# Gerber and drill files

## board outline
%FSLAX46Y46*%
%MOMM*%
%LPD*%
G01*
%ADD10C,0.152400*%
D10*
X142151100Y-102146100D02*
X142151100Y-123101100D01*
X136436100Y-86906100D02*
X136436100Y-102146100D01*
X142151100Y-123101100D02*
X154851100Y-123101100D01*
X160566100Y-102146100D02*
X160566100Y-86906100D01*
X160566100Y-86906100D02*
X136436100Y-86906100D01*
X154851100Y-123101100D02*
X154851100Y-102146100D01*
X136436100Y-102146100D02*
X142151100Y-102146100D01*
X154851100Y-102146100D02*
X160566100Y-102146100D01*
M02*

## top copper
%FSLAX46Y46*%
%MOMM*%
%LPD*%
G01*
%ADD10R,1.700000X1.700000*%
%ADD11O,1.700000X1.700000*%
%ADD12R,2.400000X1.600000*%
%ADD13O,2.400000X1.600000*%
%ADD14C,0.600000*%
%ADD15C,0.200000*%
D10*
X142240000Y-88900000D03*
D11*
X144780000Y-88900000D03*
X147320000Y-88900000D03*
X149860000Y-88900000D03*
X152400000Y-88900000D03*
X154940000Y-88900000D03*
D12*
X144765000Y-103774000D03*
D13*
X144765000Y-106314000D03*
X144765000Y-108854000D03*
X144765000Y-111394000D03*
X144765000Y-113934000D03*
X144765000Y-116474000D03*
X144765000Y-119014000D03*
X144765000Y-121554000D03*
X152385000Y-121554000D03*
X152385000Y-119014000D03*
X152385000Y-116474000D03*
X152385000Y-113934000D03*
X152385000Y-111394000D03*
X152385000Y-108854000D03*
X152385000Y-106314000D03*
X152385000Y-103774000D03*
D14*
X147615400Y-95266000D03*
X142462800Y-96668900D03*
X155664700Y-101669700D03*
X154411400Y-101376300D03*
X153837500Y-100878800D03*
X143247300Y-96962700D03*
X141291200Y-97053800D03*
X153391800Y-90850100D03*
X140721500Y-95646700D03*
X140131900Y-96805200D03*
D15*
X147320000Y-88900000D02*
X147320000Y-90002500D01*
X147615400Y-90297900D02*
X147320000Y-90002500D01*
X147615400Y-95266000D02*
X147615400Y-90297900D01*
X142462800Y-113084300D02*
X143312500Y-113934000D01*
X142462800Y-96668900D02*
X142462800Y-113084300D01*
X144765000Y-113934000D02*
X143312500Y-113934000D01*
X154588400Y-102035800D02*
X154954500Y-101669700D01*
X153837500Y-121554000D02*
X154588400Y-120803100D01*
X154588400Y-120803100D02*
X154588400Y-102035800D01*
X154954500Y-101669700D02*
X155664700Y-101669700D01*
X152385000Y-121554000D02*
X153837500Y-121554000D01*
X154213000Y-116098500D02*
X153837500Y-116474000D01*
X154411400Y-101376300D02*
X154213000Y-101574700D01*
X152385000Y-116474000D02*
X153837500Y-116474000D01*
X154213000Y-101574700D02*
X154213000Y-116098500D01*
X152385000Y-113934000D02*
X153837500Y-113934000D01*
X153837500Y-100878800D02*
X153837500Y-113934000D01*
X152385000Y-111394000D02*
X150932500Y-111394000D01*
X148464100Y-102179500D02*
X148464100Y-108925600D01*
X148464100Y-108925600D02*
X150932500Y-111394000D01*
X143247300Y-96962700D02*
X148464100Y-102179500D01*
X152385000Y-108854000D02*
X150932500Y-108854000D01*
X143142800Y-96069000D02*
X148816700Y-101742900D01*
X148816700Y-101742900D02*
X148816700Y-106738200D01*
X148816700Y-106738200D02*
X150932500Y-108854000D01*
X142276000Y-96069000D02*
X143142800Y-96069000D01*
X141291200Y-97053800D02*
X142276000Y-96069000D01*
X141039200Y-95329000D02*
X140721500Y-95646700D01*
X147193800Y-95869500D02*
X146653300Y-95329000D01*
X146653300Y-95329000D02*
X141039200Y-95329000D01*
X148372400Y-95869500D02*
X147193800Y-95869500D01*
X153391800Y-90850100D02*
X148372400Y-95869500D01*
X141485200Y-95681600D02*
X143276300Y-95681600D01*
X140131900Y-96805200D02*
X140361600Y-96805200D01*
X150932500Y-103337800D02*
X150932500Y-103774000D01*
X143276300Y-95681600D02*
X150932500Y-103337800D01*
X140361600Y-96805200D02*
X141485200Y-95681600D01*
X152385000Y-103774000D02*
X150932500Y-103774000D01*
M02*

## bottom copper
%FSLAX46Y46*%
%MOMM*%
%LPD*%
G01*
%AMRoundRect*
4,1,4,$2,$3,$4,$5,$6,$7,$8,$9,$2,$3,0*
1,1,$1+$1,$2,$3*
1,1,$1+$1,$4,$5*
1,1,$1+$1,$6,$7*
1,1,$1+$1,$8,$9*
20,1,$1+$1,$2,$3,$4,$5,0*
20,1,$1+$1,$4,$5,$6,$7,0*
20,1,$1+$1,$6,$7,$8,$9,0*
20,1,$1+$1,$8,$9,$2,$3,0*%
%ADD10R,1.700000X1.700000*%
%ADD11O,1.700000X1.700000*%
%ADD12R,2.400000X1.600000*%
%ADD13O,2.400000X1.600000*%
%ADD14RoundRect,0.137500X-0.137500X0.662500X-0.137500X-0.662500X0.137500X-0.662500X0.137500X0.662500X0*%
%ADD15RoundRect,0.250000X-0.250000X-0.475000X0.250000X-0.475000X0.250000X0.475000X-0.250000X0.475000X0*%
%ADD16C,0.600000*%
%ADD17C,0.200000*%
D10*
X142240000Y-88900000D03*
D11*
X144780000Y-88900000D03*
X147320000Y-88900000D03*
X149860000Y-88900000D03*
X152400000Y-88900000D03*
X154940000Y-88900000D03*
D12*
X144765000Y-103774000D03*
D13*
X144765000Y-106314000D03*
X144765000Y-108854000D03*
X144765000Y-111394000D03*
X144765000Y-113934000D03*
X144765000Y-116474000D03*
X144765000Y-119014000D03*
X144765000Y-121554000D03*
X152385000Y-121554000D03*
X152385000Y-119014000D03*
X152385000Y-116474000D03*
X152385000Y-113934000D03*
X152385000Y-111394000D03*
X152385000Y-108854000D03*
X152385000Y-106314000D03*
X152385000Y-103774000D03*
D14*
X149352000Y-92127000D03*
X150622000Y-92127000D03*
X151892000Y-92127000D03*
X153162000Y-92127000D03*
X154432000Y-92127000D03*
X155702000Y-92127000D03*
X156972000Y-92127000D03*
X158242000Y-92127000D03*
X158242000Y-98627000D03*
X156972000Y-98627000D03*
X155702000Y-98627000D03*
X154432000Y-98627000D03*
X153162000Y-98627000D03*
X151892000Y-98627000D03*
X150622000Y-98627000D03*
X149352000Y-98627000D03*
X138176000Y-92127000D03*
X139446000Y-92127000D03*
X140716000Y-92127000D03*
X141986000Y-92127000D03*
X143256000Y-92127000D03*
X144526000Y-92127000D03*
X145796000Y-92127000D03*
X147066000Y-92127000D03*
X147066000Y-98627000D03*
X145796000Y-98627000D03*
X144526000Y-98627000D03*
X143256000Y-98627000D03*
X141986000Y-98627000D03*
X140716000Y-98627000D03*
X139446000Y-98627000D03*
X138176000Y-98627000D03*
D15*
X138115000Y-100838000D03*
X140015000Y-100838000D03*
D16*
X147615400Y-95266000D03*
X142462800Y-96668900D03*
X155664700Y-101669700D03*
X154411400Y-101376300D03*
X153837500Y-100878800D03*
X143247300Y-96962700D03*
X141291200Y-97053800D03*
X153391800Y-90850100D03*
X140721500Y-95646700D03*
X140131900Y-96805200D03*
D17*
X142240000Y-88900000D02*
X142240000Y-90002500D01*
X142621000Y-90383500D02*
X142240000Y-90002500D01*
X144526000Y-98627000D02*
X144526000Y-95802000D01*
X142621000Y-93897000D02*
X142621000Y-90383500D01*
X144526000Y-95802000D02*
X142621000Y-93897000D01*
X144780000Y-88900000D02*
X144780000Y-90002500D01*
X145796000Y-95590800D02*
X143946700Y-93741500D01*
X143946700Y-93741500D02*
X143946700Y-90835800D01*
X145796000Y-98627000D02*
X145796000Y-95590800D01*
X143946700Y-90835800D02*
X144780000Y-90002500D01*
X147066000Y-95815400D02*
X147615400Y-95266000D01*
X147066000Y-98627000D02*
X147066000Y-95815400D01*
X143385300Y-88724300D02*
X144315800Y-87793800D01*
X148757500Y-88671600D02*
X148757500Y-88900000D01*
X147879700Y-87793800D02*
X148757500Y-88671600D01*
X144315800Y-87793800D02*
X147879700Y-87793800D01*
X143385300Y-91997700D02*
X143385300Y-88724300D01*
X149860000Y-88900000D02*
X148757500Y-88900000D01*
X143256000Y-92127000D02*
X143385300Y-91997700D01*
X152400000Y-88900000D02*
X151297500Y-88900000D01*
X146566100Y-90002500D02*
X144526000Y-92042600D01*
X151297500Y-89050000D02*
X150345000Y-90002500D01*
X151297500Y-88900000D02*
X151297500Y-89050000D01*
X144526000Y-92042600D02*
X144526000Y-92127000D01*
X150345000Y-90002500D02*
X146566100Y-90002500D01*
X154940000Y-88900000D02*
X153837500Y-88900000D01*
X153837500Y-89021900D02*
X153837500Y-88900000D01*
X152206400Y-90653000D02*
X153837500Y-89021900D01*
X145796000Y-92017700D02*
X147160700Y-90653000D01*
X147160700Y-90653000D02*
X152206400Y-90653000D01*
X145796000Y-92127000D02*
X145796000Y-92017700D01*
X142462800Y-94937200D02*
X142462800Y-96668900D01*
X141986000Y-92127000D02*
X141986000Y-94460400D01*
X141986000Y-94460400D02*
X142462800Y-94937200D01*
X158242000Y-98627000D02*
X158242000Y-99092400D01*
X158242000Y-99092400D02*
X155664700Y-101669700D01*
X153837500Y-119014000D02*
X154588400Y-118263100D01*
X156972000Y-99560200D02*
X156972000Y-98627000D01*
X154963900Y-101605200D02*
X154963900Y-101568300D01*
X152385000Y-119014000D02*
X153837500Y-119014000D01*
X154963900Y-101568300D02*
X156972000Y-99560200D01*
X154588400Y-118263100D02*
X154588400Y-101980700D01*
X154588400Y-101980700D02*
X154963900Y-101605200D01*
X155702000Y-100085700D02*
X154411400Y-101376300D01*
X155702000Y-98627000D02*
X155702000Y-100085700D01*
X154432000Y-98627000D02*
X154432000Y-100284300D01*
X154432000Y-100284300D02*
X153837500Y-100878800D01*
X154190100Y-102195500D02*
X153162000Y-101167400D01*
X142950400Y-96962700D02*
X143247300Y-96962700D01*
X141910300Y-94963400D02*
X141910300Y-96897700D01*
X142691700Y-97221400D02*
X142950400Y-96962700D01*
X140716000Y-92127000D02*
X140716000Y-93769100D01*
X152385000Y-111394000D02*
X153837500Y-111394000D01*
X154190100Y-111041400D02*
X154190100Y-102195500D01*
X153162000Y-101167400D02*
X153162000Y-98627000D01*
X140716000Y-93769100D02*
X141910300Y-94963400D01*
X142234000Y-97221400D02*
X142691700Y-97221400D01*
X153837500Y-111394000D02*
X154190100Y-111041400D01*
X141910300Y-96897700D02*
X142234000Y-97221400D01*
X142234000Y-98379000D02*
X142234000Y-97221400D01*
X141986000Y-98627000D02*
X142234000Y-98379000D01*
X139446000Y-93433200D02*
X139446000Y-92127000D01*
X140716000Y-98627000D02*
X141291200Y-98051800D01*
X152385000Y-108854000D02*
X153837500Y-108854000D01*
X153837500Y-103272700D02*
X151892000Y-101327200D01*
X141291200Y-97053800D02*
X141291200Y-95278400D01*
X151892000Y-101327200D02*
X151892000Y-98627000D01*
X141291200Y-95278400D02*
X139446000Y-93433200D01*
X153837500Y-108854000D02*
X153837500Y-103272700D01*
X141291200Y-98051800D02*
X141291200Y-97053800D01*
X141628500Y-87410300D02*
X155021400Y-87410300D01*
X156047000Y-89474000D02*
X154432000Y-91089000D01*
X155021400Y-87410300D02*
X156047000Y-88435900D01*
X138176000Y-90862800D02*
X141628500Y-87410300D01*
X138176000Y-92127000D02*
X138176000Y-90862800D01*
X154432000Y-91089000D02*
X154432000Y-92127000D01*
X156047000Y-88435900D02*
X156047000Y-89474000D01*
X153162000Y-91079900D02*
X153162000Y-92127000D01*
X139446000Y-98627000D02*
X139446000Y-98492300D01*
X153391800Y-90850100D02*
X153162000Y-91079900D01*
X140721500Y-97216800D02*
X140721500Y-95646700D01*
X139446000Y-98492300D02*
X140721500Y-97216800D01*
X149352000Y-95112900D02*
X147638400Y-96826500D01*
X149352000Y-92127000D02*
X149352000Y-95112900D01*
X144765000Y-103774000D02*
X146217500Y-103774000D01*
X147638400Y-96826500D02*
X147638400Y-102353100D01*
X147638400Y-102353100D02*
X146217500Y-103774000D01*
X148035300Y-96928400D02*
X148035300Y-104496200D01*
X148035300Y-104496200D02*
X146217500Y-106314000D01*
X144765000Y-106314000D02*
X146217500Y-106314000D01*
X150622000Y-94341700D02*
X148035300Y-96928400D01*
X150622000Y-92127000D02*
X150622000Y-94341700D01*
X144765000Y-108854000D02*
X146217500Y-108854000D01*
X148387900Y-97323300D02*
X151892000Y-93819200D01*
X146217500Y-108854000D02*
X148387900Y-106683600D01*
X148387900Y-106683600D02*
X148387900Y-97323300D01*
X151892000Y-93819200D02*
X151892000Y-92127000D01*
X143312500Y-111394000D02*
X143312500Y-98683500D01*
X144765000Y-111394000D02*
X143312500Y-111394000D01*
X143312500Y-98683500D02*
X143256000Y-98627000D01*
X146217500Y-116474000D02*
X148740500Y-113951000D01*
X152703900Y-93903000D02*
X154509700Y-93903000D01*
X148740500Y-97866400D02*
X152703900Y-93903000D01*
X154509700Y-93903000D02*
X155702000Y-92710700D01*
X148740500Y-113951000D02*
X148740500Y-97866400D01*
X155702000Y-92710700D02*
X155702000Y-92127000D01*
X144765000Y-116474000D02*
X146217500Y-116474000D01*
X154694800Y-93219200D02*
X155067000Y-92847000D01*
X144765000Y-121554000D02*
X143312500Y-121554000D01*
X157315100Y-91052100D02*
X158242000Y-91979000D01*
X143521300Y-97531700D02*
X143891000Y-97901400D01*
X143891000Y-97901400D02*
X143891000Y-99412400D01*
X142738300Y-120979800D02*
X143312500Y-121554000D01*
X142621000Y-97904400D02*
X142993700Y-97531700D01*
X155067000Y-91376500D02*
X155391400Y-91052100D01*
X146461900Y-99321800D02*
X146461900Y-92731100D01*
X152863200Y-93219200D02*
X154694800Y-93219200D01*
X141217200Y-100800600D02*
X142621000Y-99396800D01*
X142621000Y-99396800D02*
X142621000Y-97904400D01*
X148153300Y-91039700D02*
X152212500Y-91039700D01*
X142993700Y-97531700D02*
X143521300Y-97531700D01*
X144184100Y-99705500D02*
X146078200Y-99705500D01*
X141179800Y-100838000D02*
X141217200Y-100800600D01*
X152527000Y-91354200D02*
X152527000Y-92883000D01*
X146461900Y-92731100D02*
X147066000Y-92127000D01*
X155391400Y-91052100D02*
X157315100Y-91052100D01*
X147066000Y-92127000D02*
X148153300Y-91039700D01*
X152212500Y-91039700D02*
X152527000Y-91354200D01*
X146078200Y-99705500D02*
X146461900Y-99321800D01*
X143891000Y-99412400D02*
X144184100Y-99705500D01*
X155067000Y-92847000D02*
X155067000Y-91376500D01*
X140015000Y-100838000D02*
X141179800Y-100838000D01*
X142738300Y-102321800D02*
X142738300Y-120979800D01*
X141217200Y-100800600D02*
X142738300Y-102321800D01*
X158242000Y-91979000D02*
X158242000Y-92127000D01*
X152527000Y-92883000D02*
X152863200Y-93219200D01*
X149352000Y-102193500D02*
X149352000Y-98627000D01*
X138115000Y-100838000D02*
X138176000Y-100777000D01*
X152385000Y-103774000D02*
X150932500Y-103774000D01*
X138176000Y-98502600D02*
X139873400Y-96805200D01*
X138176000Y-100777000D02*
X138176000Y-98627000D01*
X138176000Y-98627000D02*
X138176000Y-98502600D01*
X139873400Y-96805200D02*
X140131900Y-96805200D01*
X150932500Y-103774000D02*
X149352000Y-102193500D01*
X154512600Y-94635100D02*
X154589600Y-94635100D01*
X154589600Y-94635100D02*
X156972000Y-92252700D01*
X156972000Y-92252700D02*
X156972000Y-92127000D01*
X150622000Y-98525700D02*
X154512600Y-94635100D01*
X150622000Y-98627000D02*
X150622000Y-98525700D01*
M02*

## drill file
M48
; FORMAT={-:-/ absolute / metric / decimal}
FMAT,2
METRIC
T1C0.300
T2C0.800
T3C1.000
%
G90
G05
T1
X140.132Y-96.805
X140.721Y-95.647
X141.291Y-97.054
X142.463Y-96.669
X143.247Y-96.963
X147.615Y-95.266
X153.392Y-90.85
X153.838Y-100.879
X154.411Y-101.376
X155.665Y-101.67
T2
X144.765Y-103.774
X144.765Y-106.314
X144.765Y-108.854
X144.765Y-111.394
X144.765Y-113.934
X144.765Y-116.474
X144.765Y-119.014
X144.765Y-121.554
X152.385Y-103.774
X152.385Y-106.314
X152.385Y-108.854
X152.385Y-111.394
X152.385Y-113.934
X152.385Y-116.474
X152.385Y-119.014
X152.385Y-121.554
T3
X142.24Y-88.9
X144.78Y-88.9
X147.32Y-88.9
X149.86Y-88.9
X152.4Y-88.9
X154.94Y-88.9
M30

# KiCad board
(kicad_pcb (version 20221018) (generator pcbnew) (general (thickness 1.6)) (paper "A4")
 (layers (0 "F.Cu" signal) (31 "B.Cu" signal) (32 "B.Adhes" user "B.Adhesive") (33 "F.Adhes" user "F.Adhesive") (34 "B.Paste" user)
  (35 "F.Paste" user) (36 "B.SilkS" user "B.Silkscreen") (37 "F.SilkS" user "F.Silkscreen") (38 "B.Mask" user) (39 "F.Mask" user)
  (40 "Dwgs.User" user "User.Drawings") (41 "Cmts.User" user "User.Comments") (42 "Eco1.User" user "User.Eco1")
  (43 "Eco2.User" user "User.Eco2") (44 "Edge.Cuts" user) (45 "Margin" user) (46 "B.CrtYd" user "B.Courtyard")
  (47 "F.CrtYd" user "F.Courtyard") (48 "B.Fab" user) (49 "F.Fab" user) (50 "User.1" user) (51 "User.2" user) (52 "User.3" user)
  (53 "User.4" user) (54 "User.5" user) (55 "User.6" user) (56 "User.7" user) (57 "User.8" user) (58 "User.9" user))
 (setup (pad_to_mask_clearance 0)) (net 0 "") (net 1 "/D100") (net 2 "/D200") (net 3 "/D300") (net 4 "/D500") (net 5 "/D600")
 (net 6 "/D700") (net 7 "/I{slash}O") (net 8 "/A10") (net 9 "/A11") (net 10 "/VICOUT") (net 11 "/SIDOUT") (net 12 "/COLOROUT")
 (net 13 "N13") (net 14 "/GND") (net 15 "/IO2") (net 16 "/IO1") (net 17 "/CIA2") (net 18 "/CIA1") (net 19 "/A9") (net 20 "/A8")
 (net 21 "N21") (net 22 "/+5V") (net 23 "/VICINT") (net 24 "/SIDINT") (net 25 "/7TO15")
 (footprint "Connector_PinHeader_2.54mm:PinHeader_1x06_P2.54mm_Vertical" (layer "F.Cu") (at 142.24 88.9 90)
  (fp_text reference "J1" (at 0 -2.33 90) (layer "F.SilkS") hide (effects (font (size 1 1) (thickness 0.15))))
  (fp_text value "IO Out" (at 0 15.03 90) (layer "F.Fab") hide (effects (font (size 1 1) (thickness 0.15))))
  (pad "1" thru_hole rect (at 0 0 90) (size 1.7 1.7) (drill 1) (layers "*.Cu" "*.Mask") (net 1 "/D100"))
  (pad "2" thru_hole oval (at 0 2.54 90) (size 1.7 1.7) (drill 1) (layers "*.Cu" "*.Mask") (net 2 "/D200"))
  (pad "3" thru_hole oval (at 0 5.08 90) (size 1.7 1.7) (drill 1) (layers "*.Cu" "*.Mask") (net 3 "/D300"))
  (pad "4" thru_hole oval (at 0 7.62 90) (size 1.7 1.7) (drill 1) (layers "*.Cu" "*.Mask") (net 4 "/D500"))
  (pad "5" thru_hole oval (at 0 10.16 90) (size 1.7 1.7) (drill 1) (layers "*.Cu" "*.Mask") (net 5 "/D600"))
  (pad "6" thru_hole oval (at 0 12.7 90) (size 1.7 1.7) (drill 1) (layers "*.Cu" "*.Mask") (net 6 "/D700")))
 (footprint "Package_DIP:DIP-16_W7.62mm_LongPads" (layer "F.Cu") (at 144.765 103.774)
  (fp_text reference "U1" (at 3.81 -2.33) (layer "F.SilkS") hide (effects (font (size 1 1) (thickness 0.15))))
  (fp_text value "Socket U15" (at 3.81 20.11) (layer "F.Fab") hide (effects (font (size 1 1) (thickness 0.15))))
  (pad "1" thru_hole rect (at 0 0) (size 2.4 1.6) (drill 0.8) (layers "*.Cu" "*.Mask") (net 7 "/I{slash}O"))
  (pad "2" thru_hole oval (at 0 2.54) (size 2.4 1.6) (drill 0.8) (layers "*.Cu" "*.Mask") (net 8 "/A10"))
  (pad "3" thru_hole oval (at 0 5.08) (size 2.4 1.6) (drill 0.8) (layers "*.Cu" "*.Mask") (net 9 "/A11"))
  (pad "4" thru_hole oval (at 0 7.62) (size 2.4 1.6) (drill 0.8) (layers "*.Cu" "*.Mask") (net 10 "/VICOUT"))
  (pad "5" thru_hole oval (at 0 10.16) (size 2.4 1.6) (drill 0.8) (layers "*.Cu" "*.Mask") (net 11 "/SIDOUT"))
  (pad "6" thru_hole oval (at 0 12.7) (size 2.4 1.6) (drill 0.8) (layers "*.Cu" "*.Mask") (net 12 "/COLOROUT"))
  (pad "7" thru_hole oval (at 0 15.24) (size 2.4 1.6) (drill 0.8) (layers "*.Cu" "*.Mask") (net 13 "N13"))
  (pad "8" thru_hole oval (at 0 17.78) (size 2.4 1.6) (drill 0.8) (layers "*.Cu" "*.Mask") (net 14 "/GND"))
  (pad "9" thru_hole oval (at 7.62 17.78) (size 2.4 1.6) (drill 0.8) (layers "*.Cu" "*.Mask") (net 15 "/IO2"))
  (pad "10" thru_hole oval (at 7.62 15.24) (size 2.4 1.6) (drill 0.8) (layers "*.Cu" "*.Mask") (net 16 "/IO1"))
  (pad "11" thru_hole oval (at 7.62 12.7) (size 2.4 1.6) (drill 0.8) (layers "*.Cu" "*.Mask") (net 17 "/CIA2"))
  (pad "12" thru_hole oval (at 7.62 10.16) (size 2.4 1.6) (drill 0.8) (layers "*.Cu" "*.Mask") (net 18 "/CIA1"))
  (pad "13" thru_hole oval (at 7.62 7.62) (size 2.4 1.6) (drill 0.8) (layers "*.Cu" "*.Mask") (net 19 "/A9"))
  (pad "14" thru_hole oval (at 7.62 5.08) (size 2.4 1.6) (drill 0.8) (layers "*.Cu" "*.Mask") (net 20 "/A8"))
  (pad "15" thru_hole oval (at 7.62 2.54) (size 2.4 1.6) (drill 0.8) (layers "*.Cu" "*.Mask") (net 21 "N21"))
  (pad "16" thru_hole oval (at 7.62 0) (size 2.4 1.6) (drill 0.8) (layers "*.Cu" "*.Mask") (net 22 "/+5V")))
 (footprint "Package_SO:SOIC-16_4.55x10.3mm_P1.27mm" (layer "B.Cu") (at 153.797 95.377 -90)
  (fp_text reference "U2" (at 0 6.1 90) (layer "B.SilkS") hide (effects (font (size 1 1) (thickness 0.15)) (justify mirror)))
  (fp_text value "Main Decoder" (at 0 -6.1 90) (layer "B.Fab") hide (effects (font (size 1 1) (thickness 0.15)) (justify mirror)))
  (pad "1" smd roundrect (at -3.25 4.445 270) (size 1.6 0.55) (layers "B.Cu" "B.Paste" "B.Mask") (roundrect_rratio 0.25)
   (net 7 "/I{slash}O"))
  (pad "2" smd roundrect (at -3.25 3.175 270) (size 1.6 0.55) (layers "B.Cu" "B.Paste" "B.Mask") (roundrect_rratio 0.25) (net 8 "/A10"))
  (pad "3" smd roundrect (at -3.25 1.905 270) (size 1.6 0.55) (layers "B.Cu" "B.Paste" "B.Mask") (roundrect_rratio 0.25) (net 9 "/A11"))
  (pad "4" smd roundrect (at -3.25 0.635 270) (size 1.6 0.55) (layers "B.Cu" "B.Paste" "B.Mask") (roundrect_rratio 0.25) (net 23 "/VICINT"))
  (pad "5" smd roundrect (at -3.25 -0.635 270) (size 1.6 0.55) (layers "B.Cu" "B.Paste" "B.Mask") (roundrect_rratio 0.25) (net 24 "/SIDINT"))
  (pad "6" smd roundrect (at -3.25 -1.905 270) (size 1.6 0.55) (layers "B.Cu" "B.Paste" "B.Mask") (roundrect_rratio 0.25)
   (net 12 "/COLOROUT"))
  (pad "7" smd roundrect (at -3.25 -3.175 270) (size 1.6 0.55) (layers "B.Cu" "B.Paste" "B.Mask") (roundrect_rratio 0.25) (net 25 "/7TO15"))
  (pad "8" smd roundrect (at -3.25 -4.445 270) (size 1.6 0.55) (layers "B.Cu" "B.Paste" "B.Mask") (roundrect_rratio 0.25) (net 14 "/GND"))
  (pad "9" smd roundrect (at 3.25 -4.445 270) (size 1.6 0.55) (layers "B.Cu" "B.Paste" "B.Mask") (roundrect_rratio 0.25) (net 15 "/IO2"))
  (pad "10" smd roundrect (at 3.25 -3.175 270) (size 1.6 0.55) (layers "B.Cu" "B.Paste" "B.Mask") (roundrect_rratio 0.25) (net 16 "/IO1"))
  (pad "11" smd roundrect (at 3.25 -1.905 270) (size 1.6 0.55) (layers "B.Cu" "B.Paste" "B.Mask") (roundrect_rratio 0.25) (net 17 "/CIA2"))
  (pad "12" smd roundrect (at 3.25 -0.635 270) (size 1.6 0.55) (layers "B.Cu" "B.Paste" "B.Mask") (roundrect_rratio 0.25) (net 18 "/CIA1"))
  (pad "13" smd roundrect (at 3.25 0.635 270) (size 1.6 0.55) (layers "B.Cu" "B.Paste" "B.Mask") (roundrect_rratio 0.25) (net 19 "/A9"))
  (pad "14" smd roundrect (at 3.25 1.905 270) (size 1.6 0.55) (layers "B.Cu" "B.Paste" "B.Mask") (roundrect_rratio 0.25) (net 20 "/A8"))
  (pad "15" smd roundrect (at 3.25 3.175 270) (size 1.6 0.55) (layers "B.Cu" "B.Paste" "B.Mask") (roundrect_rratio 0.25) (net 25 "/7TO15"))
  (pad "16" smd roundrect (at 3.25 4.445 270) (size 1.6 0.55) (layers "B.Cu" "B.Paste" "B.Mask") (roundrect_rratio 0.25) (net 22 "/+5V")))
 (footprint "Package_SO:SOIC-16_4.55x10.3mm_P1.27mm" (layer "B.Cu") (at 142.621 95.377 -90)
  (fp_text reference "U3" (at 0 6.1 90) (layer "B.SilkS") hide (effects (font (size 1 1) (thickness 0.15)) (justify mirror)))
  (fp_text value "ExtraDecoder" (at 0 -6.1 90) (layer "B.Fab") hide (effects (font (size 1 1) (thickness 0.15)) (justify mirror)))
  (pad "1" smd roundrect (at -3.25 4.445 270) (size 1.6 0.55) (layers "B.Cu" "B.Paste" "B.Mask") (roundrect_rratio 0.25) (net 24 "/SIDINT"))
  (pad "2" smd roundrect (at -3.25 3.175 270) (size 1.6 0.55) (layers "B.Cu" "B.Paste" "B.Mask") (roundrect_rratio 0.25) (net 20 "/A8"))
  (pad "3" smd roundrect (at -3.25 1.905 270) (size 1.6 0.55) (layers "B.Cu" "B.Paste" "B.Mask") (roundrect_rratio 0.25) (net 19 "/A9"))
  (pad "4" smd roundrect (at -3.25 0.635 270) (size 1.6 0.55) (layers "B.Cu" "B.Paste" "B.Mask") (roundrect_rratio 0.25) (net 11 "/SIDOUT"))
  (pad "5" smd roundrect (at -3.25 -0.635 270) (size 1.6 0.55) (layers "B.Cu" "B.Paste" "B.Mask") (roundrect_rratio 0.25) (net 4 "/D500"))
  (pad "6" smd roundrect (at -3.25 -1.905 270) (size 1.6 0.55) (layers "B.Cu" "B.Paste" "B.Mask") (roundrect_rratio 0.25) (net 5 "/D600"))
  (pad "7" smd roundrect (at -3.25 -3.175 270) (size 1.6 0.55) (layers "B.Cu" "B.Paste" "B.Mask") (roundrect_rratio 0.25) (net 6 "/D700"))
  (pad "8" smd roundrect (at -3.25 -4.445 270) (size 1.6 0.55) (layers "B.Cu" "B.Paste" "B.Mask") (roundrect_rratio 0.25) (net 14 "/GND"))
  (pad "9" smd roundrect (at 3.25 -4.445 270) (size 1.6 0.55) (layers "B.Cu" "B.Paste" "B.Mask") (roundrect_rratio 0.25) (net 3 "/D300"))
  (pad "10" smd roundrect (at 3.25 -3.175 270) (size 1.6 0.55) (layers "B.Cu" "B.Paste" "B.Mask") (roundrect_rratio 0.25) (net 2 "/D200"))
  (pad "11" smd roundrect (at 3.25 -1.905 270) (size 1.6 0.55) (layers "B.Cu" "B.Paste" "B.Mask") (roundrect_rratio 0.25) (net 1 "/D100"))
  (pad "12" smd roundrect (at 3.25 -0.635 270) (size 1.6 0.55) (layers "B.Cu" "B.Paste" "B.Mask") (roundrect_rratio 0.25) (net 10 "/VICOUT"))
  (pad "13" smd roundrect (at 3.25 0.635 270) (size 1.6 0.55) (layers "B.Cu" "B.Paste" "B.Mask") (roundrect_rratio 0.25) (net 19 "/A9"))
  (pad "14" smd roundrect (at 3.25 1.905 270) (size 1.6 0.55) (layers "B.Cu" "B.Paste" "B.Mask") (roundrect_rratio 0.25) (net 20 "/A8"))
  (pad "15" smd roundrect (at 3.25 3.175 270) (size 1.6 0.55) (layers "B.Cu" "B.Paste" "B.Mask") (roundrect_rratio 0.25) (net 23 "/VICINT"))
  (pad "16" smd roundrect (at 3.25 4.445 270) (size 1.6 0.55) (layers "B.Cu" "B.Paste" "B.Mask") (roundrect_rratio 0.25) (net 22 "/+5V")))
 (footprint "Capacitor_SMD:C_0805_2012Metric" (layer "B.Cu") (at 139.065 100.838)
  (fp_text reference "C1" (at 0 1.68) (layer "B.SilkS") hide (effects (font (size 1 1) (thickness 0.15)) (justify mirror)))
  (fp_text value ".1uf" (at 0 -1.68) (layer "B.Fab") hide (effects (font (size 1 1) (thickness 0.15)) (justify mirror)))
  (pad "1" smd roundrect (at -0.95 0) (size 1 1.45) (layers "B.Cu" "B.Paste" "B.Mask") (roundrect_rratio 0.25) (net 22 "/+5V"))
  (pad "2" smd roundrect (at 0.95 0) (size 1 1.45) (layers "B.Cu" "B.Paste" "B.Mask") (roundrect_rratio 0.25) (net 14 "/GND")))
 (gr_line (start 142.1511 102.1461) (end 142.1511 123.1011) (stroke (width 0.1524) (type solid)) (layer "Edge.Cuts"))
 (gr_line (start 136.4361 86.9061) (end 136.4361 102.1461) (stroke (width 0.1524) (type solid)) (layer "Edge.Cuts"))
 (gr_line (start 142.1511 123.1011) (end 154.8511 123.1011) (stroke (width 0.1524) (type solid)) (layer "Edge.Cuts"))
 (gr_line (start 160.5661 102.1461) (end 160.5661 86.9061) (stroke (width 0.1524) (type solid)) (layer "Edge.Cuts"))
 (gr_line (start 160.5661 86.9061) (end 136.4361 86.9061) (stroke (width 0.1524) (type solid)) (layer "Edge.Cuts"))
 (gr_line (start 154.8511 123.1011) (end 154.8511 102.1461) (stroke (width 0.1524) (type solid)) (layer "Edge.Cuts"))
 (gr_line (start 136.4361 102.1461) (end 142.1511 102.1461) (stroke (width 0.1524) (type solid)) (layer "Edge.Cuts"))
 (gr_line (start 154.8511 102.1461) (end 160.5661 102.1461) (stroke (width 0.1524) (type solid)) (layer "Edge.Cuts"))
 (segment (start 142.24 88.9) (end 142.24 90.0025) (width 0.2) (layer "B.Cu") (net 1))
 (segment (start 142.621 90.3835) (end 142.24 90.0025) (width 0.2) (layer "B.Cu") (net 1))
 (segment (start 144.526 98.627) (end 144.526 95.802) (width 0.2) (layer "B.Cu") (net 1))
 (segment (start 142.621 93.897) (end 142.621 90.3835) (width 0.2) (layer "B.Cu") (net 1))
 (segment (start 144.526 95.802) (end 142.621 93.897) (width 0.2) (layer "B.Cu") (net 1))
 (segment (start 144.78 88.9) (end 144.78 90.0025) (width 0.2) (layer "B.Cu") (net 2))
 (segment (start 145.796 95.5908) (end 143.9467 93.7415) (width 0.2) (layer "B.Cu") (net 2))
 (segment (start 143.9467 93.7415) (end 143.9467 90.8358) (width 0.2) (layer "B.Cu") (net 2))
 (segment (start 145.796 98.627) (end 145.796 95.5908) (width 0.2) (layer "B.Cu") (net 2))
 (segment (start 143.9467 90.8358) (end 144.78 90.0025) (width 0.2) (layer "B.Cu") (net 2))
 (segment (start 147.32 88.9) (end 147.32 90.0025) (width 0.2) (layer "F.Cu") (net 3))
 (segment (start 147.6154 90.2979) (end 147.32 90.0025) (width 0.2) (layer "F.Cu") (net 3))
 (segment (start 147.6154 95.266) (end 147.6154 90.2979) (width 0.2) (layer "F.Cu") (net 3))
 (via (at 147.6154 95.266) (size 0.6) (drill 0.3) (layers "F.Cu" "B.Cu") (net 3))
 (segment (start 147.066 95.8154) (end 147.6154 95.266) (width 0.2) (layer "B.Cu") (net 3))
 (segment (start 147.066 98.627) (end 147.066 95.8154) (width 0.2) (layer "B.Cu") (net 3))
 (segment (start 143.3853 88.7243) (end 144.3158 87.7938) (width 0.2) (layer "B.Cu") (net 4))
 (segment (start 148.7575 88.6716) (end 148.7575 88.9) (width 0.2) (layer "B.Cu") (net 4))
 (segment (start 147.8797 87.7938) (end 148.7575 88.6716) (width 0.2) (layer "B.Cu") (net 4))
 (segment (start 144.3158 87.7938) (end 147.8797 87.7938) (width 0.2) (layer "B.Cu") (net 4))
 (segment (start 143.3853 91.9977) (end 143.3853 88.7243) (width 0.2) (layer "B.Cu") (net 4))
 (segment (start 149.86 88.9) (end 148.7575 88.9) (width 0.2) (layer "B.Cu") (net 4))
 (segment (start 143.256 92.127) (end 143.3853 91.9977) (width 0.2) (layer "B.Cu") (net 4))
 (segment (start 152.4 88.9) (end 151.2975 88.9) (width 0.2) (layer "B.Cu") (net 5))
 (segment (start 146.5661 90.0025) (end 144.526 92.0426) (width 0.2) (layer "B.Cu") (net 5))
 (segment (start 151.2975 89.05) (end 150.345 90.0025) (width 0.2) (layer "B.Cu") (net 5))
 (segment (start 151.2975 88.9) (end 151.2975 89.05) (width 0.2) (layer "B.Cu") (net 5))
 (segment (start 144.526 92.0426) (end 144.526 92.127) (width 0.2) (layer "B.Cu") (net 5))
 (segment (start 150.345 90.0025) (end 146.5661 90.0025) (width 0.2) (layer "B.Cu") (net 5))
 (segment (start 154.94 88.9) (end 153.8375 88.9) (width 0.2) (layer "B.Cu") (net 6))
 (segment (start 153.8375 89.0219) (end 153.8375 88.9) (width 0.2) (layer "B.Cu") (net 6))
 (segment (start 152.2064 90.653) (end 153.8375 89.0219) (width 0.2) (layer "B.Cu") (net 6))
 (segment (start 145.796 92.0177) (end 147.1607 90.653) (width 0.2) (layer "B.Cu") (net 6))
 (segment (start 147.1607 90.653) (end 152.2064 90.653) (width 0.2) (layer "B.Cu") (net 6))
 (segment (start 145.796 92.127) (end 145.796 92.0177) (width 0.2) (layer "B.Cu") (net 6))
 (segment (start 142.4628 113.0843) (end 143.3125 113.934) (width 0.2) (layer "F.Cu") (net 11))
 (segment (start 142.4628 96.6689) (end 142.4628 113.0843) (width 0.2) (layer "F.Cu") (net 11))
 (segment (start 144.765 113.934) (end 143.3125 113.934) (width 0.2) (layer "F.Cu") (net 11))
 (via (at 142.4628 96.6689) (size 0.6) (drill 0.3) (layers "F.Cu" "B.Cu") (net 11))
 (segment (start 142.4628 94.9372) (end 142.4628 96.6689) (width 0.2) (layer "B.Cu") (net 11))
 (segment (start 141.986 92.127) (end 141.986 94.4604) (width 0.2) (layer "B.Cu") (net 11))
 (segment (start 141.986 94.4604) (end 142.4628 94.9372) (width 0.2) (layer "B.Cu") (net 11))
 (segment (start 154.5884 102.0358) (end 154.9545 101.6697) (width 0.2) (layer "F.Cu") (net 15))
 (segment (start 153.8375 121.554) (end 154.5884 120.8031) (width 0.2) (layer "F.Cu") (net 15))
 (segment (start 154.5884 120.8031) (end 154.5884 102.0358) (width 0.2) (layer "F.Cu") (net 15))
 (segment (start 154.9545 101.6697) (end 155.6647 101.6697) (width 0.2) (layer "F.Cu") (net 15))
 (segment (start 152.385 121.554) (end 153.8375 121.554) (width 0.2) (layer "F.Cu") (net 15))
 (via (at 155.6647 101.6697) (size 0.6) (drill 0.3) (layers "F.Cu" "B.Cu") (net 15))
 (segment (start 158.242 98.627) (end 158.242 99.0924) (width 0.2) (layer "B.Cu") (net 15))
 (segment (start 158.242 99.0924) (end 155.6647 101.6697) (width 0.2) (layer "B.Cu") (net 15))
 (segment (start 153.8375 119.014) (end 154.5884 118.2631) (width 0.2) (layer "B.Cu") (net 16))
 (segment (start 156.972 99.5602) (end 156.972 98.627) (width 0.2) (layer "B.Cu") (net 16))
 (segment (start 154.9639 101.6052) (end 154.9639 101.5683) (width 0.2) (layer "B.Cu") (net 16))
 (segment (start 152.385 119.014) (end 153.8375 119.014) (width 0.2) (layer "B.Cu") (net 16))
 (segment (start 154.9639 101.5683) (end 156.972 99.5602) (width 0.2) (layer "B.Cu") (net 16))
 (segment (start 154.5884 118.2631) (end 154.5884 101.9807) (width 0.2) (layer "B.Cu") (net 16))
 (segment (start 154.5884 101.9807) (end 154.9639 101.6052) (width 0.2) (layer "B.Cu") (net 16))
 (segment (start 154.213 116.0985) (end 153.8375 116.474) (width 0.2) (layer "F.Cu") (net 17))
 (segment (start 154.4114 101.3763) (end 154.213 101.5747) (width 0.2) (layer "F.Cu") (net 17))
 (segment (start 152.385 116.474) (end 153.8375 116.474) (width 0.2) (layer "F.Cu") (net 17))
 (segment (start 154.213 101.5747) (end 154.213 116.0985) (width 0.2) (layer "F.Cu") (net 17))
 (via (at 154.4114 101.3763) (size 0.6) (drill 0.3) (layers "F.Cu" "B.Cu") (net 17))
 (segment (start 155.702 100.0857) (end 154.4114 101.3763) (width 0.2) (layer "B.Cu") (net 17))
 (segment (start 155.702 98.627) (end 155.702 100.0857) (width 0.2) (layer "B.Cu") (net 17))
 (segment (start 152.385 113.934) (end 153.8375 113.934) (width 0.2) (layer "F.Cu") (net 18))
 (segment (start 153.8375 100.8788) (end 153.8375 113.934) (width 0.2) (layer "F.Cu") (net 18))
 (via (at 153.8375 100.8788) (size 0.6) (drill 0.3) (layers "F.Cu" "B.Cu") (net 18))
 (segment (start 154.432 98.627) (end 154.432 100.2843) (width 0.2) (layer "B.Cu") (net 18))
 (segment (start 154.432 100.2843) (end 153.8375 100.8788) (width 0.2) (layer "B.Cu") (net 18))
 (segment (start 152.385 111.394) (end 150.9325 111.394) (width 0.2) (layer "F.Cu") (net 19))
 (segment (start 148.4641 102.1795) (end 148.4641 108.9256) (width 0.2) (layer "F.Cu") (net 19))
 (segment (start 148.4641 108.9256) (end 150.9325 111.394) (width 0.2) (layer "F.Cu") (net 19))
 (segment (start 143.2473 96.9627) (end 148.4641 102.1795) (width 0.2) (layer "F.Cu") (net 19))
 (via (at 143.2473 96.9627) (size 0.6) (drill 0.3) (layers "F.Cu" "B.Cu") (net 19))
 (segment (start 154.1901 102.1955) (end 153.162 101.1674) (width 0.2) (layer "B.Cu") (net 19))
 (segment (start 142.9504 96.9627) (end 143.2473 96.9627) (width 0.2) (layer "B.Cu") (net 19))
 (segment (start 141.9103 94.9634) (end 141.9103 96.8977) (width 0.2) (layer "B.Cu") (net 19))
 (segment (start 142.6917 97.2214) (end 142.9504 96.9627) (width 0.2) (layer "B.Cu") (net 19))
 (segment (start 140.716 92.127) (end 140.716 93.7691) (width 0.2) (layer "B.Cu") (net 19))
 (segment (start 152.385 111.394) (end 153.8375 111.394) (width 0.2) (layer "B.Cu") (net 19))
 (segment (start 154.1901 111.0414) (end 154.1901 102.1955) (width 0.2) (layer "B.Cu") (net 19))
 (segment (start 153.162 101.1674) (end 153.162 98.627) (width 0.2) (layer "B.Cu") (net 19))
 (segment (start 140.716 93.7691) (end 141.9103 94.9634) (width 0.2) (layer "B.Cu") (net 19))
 (segment (start 142.234 97.2214) (end 142.6917 97.2214) (width 0.2) (layer "B.Cu") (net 19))
 (segment (start 153.8375 111.394) (end 154.1901 111.0414) (width 0.2) (layer "B.Cu") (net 19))
 (segment (start 141.9103 96.8977) (end 142.234 97.2214) (width 0.2) (layer "B.Cu") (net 19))
 (segment (start 142.234 98.379) (end 142.234 97.2214) (width 0.2) (layer "B.Cu") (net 19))
 (segment (start 141.986 98.627) (end 142.234 98.379) (width 0.2) (layer "B.Cu") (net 19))
 (segment (start 152.385 108.854) (end 150.9325 108.854) (width 0.2) (layer "F.Cu") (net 20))
 (segment (start 143.1428 96.069) (end 148.8167 101.7429) (width 0.2) (layer "F.Cu") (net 20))
 (segment (start 148.8167 101.7429) (end 148.8167 106.7382) (width 0.2) (layer "F.Cu") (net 20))
 (segment (start 148.8167 106.7382) (end 150.9325 108.854) (width 0.2) (layer "F.Cu") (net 20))
 (segment (start 142.276 96.069) (end 143.1428 96.069) (width 0.2) (layer "F.Cu") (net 20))
 (segment (start 141.2912 97.0538) (end 142.276 96.069) (width 0.2) (layer "F.Cu") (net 20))
 (via (at 141.2912 97.0538) (size 0.6) (drill 0.3) (layers "F.Cu" "B.Cu") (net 20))
 (segment (start 139.446 93.4332) (end 139.446 92.127) (width 0.2) (layer "B.Cu") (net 20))
 (segment (start 140.716 98.627) (end 141.2912 98.0518) (width 0.2) (layer "B.Cu") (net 20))
 (segment (start 152.385 108.854) (end 153.8375 108.854) (width 0.2) (layer "B.Cu") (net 20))
 (segment (start 153.8375 103.2727) (end 151.892 101.3272) (width 0.2) (layer "B.Cu") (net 20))
 (segment (start 141.2912 97.0538) (end 141.2912 95.2784) (width 0.2) (layer "B.Cu") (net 20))
 (segment (start 151.892 101.3272) (end 151.892 98.627) (width 0.2) (layer "B.Cu") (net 20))
 (segment (start 141.2912 95.2784) (end 139.446 93.4332) (width 0.2) (layer "B.Cu") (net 20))
 (segment (start 153.8375 108.854) (end 153.8375 103.2727) (width 0.2) (layer "B.Cu") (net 20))
 (segment (start 141.2912 98.0518) (end 141.2912 97.0538) (width 0.2) (layer "B.Cu") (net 20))
 (segment (start 141.6285 87.4103) (end 155.0214 87.4103) (width 0.2) (layer "B.Cu") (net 24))
 (segment (start 156.047 89.474) (end 154.432 91.089) (width 0.2) (layer "B.Cu") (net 24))
 (segment (start 155.0214 87.4103) (end 156.047 88.4359) (width 0.2) (layer "B.Cu") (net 24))
 (segment (start 138.176 90.8628) (end 141.6285 87.4103) (width 0.2) (layer "B.Cu") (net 24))
 (segment (start 138.176 92.127) (end 138.176 90.8628) (width 0.2) (layer "B.Cu") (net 24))
 (segment (start 154.432 91.089) (end 154.432 92.127) (width 0.2) (layer "B.Cu") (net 24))
 (segment (start 156.047 88.4359) (end 156.047 89.474) (width 0.2) (layer "B.Cu") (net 24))
 (segment (start 141.0392 95.329) (end 140.7215 95.6467) (width 0.2) (layer "F.Cu") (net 23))
 (segment (start 147.1938 95.8695) (end 146.6533 95.329) (width 0.2) (layer "F.Cu") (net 23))
 (segment (start 146.6533 95.329) (end 141.0392 95.329) (width 0.2) (layer "F.Cu") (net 23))
 (segment (start 148.3724 95.8695) (end 147.1938 95.8695) (width 0.2) (layer "F.Cu") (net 23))
 (segment (start 153.3918 90.8501) (end 148.3724 95.8695) (width 0.2) (layer "F.Cu") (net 23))
 (via (at 153.3918 90.8501) (size 0.6) (drill 0.3) (layers "F.Cu" "B.Cu") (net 23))
 (via (at 140.7215 95.6467) (size 0.6) (drill 0.3) (layers "F.Cu" "B.Cu") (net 23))
 (segment (start 153.162 91.0799) (end 153.162 92.127) (width 0.2) (layer "B.Cu") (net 23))
 (segment (start 139.446 98.627) (end 139.446 98.4923) (width 0.2) (layer "B.Cu") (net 23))
 (segment (start 153.3918 90.8501) (end 153.162 91.0799) (width 0.2) (layer "B.Cu") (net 23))
 (segment (start 140.7215 97.2168) (end 140.7215 95.6467) (width 0.2) (layer "B.Cu") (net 23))
 (segment (start 139.446 98.4923) (end 140.7215 97.2168) (width 0.2) (layer "B.Cu") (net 23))
 (segment (start 149.352 95.1129) (end 147.6384 96.8265) (width 0.2) (layer "B.Cu") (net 7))
 (segment (start 149.352 92.127) (end 149.352 95.1129) (width 0.2) (layer "B.Cu") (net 7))
 (segment (start 144.765 103.774) (end 146.2175 103.774) (width 0.2) (layer "B.Cu") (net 7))
 (segment (start 147.6384 96.8265) (end 147.6384 102.3531) (width 0.2) (layer "B.Cu") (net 7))
 (segment (start 147.6384 102.3531) (end 146.2175 103.774) (width 0.2) (layer "B.Cu") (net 7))
 (segment (start 148.0353 96.9284) (end 148.0353 104.4962) (width 0.2) (layer "B.Cu") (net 8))
 (segment (start 148.0353 104.4962) (end 146.2175 106.314) (width 0.2) (layer "B.Cu") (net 8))
 (segment (start 144.765 106.314) (end 146.2175 106.314) (width 0.2) (layer "B.Cu") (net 8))
 (segment (start 150.622 94.3417) (end 148.0353 96.9284) (width 0.2) (layer "B.Cu") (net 8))
 (segment (start 150.622 92.127) (end 150.622 94.3417) (width 0.2) (layer "B.Cu") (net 8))
 (segment (start 144.765 108.854) (end 146.2175 108.854) (width 0.2) (layer "B.Cu") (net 9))
 (segment (start 148.3879 97.3233) (end 151.892 93.8192) (width 0.2) (layer "B.Cu") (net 9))
 (segment (start 146.2175 108.854) (end 148.3879 106.6836) (width 0.2) (layer "B.Cu") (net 9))
 (segment (start 148.3879 106.6836) (end 148.3879 97.3233) (width 0.2) (layer "B.Cu") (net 9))
 (segment (start 151.892 93.8192) (end 151.892 92.127) (width 0.2) (layer "B.Cu") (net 9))
 (segment (start 143.3125 111.394) (end 143.3125 98.6835) (width 0.2) (layer "B.Cu") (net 10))
 (segment (start 144.765 111.394) (end 143.3125 111.394) (width 0.2) (layer "B.Cu") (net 10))
 (segment (start 143.3125 98.6835) (end 143.256 98.627) (width 0.2) (layer "B.Cu") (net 10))
 (segment (start 146.2175 116.474) (end 148.7405 113.951) (width 0.2) (layer "B.Cu") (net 12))
 (segment (start 152.7039 93.903) (end 154.5097 93.903) (width 0.2) (layer "B.Cu") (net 12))
 (segment (start 148.7405 97.8664) (end 152.7039 93.903) (width 0.2) (layer "B.Cu") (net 12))
 (segment (start 154.5097 93.903) (end 155.702 92.7107) (width 0.2) (layer "B.Cu") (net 12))
 (segment (start 148.7405 113.951) (end 148.7405 97.8664) (width 0.2) (layer "B.Cu") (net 12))
 (segment (start 155.702 92.7107) (end 155.702 92.127) (width 0.2) (layer "B.Cu") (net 12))
 (segment (start 144.765 116.474) (end 146.2175 116.474) (width 0.2) (layer "B.Cu") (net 12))
 (segment (start 154.6948 93.2192) (end 155.067 92.847) (width 0.2) (layer "B.Cu") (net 14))
 (segment (start 144.765 121.554) (end 143.3125 121.554) (width 0.2) (layer "B.Cu") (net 14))
 (segment (start 157.3151 91.0521) (end 158.242 91.979) (width 0.2) (layer "B.Cu") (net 14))
 (segment (start 143.5213 97.5317) (end 143.891 97.9014) (width 0.2) (layer "B.Cu") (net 14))
 (segment (start 143.891 97.9014) (end 143.891 99.4124) (width 0.2) (layer "B.Cu") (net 14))
 (segment (start 142.7383 120.9798) (end 143.3125 121.554) (width 0.2) (layer "B.Cu") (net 14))
 (segment (start 142.621 97.9044) (end 142.9937 97.5317) (width 0.2) (layer "B.Cu") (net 14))
 (segment (start 155.067 91.3765) (end 155.3914 91.0521) (width 0.2) (layer "B.Cu") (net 14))
 (segment (start 146.4619 99.3218) (end 146.4619 92.7311) (width 0.2) (layer "B.Cu") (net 14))
 (segment (start 152.8632 93.2192) (end 154.6948 93.2192) (width 0.2) (layer "B.Cu") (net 14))
 (segment (start 141.2172 100.8006) (end 142.621 99.3968) (width 0.2) (layer "B.Cu") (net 14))
 (segment (start 142.621 99.3968) (end 142.621 97.9044) (width 0.2) (layer "B.Cu") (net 14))
 (segment (start 148.1533 91.0397) (end 152.2125 91.0397) (width 0.2) (layer "B.Cu") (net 14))
 (segment (start 142.9937 97.5317) (end 143.5213 97.5317) (width 0.2) (layer "B.Cu") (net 14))
 (segment (start 144.1841 99.7055) (end 146.0782 99.7055) (width 0.2) (layer "B.Cu") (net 14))
 (segment (start 141.1798 100.838) (end 141.2172 100.8006) (width 0.2) (layer "B.Cu") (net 14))
 (segment (start 152.527 91.3542) (end 152.527 92.883) (width 0.2) (layer "B.Cu") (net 14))
 (segment (start 146.4619 92.7311) (end 147.066 92.127) (width 0.2) (layer "B.Cu") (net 14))
 (segment (start 155.3914 91.0521) (end 157.3151 91.0521) (width 0.2) (layer "B.Cu") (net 14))
 (segment (start 147.066 92.127) (end 148.1533 91.0397) (width 0.2) (layer "B.Cu") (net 14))
 (segment (start 152.2125 91.0397) (end 152.527 91.3542) (width 0.2) (layer "B.Cu") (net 14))
 (segment (start 146.0782 99.7055) (end 146.4619 99.3218) (width 0.2) (layer "B.Cu") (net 14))
 (segment (start 143.891 99.4124) (end 144.1841 99.7055) (width 0.2) (layer "B.Cu") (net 14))
 (segment (start 155.067 92.847) (end 155.067 91.3765) (width 0.2) (layer "B.Cu") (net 14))
 (segment (start 140.015 100.838) (end 141.1798 100.838) (width 0.2) (layer "B.Cu") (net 14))
 (segment (start 142.7383 102.3218) (end 142.7383 120.9798) (width 0.2) (layer "B.Cu") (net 14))
 (segment (start 141.2172 100.8006) (end 142.7383 102.3218) (width 0.2) (layer "B.Cu") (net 14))
 (segment (start 158.242 91.979) (end 158.242 92.127) (width 0.2) (layer "B.Cu") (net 14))
 (segment (start 152.527 92.883) (end 152.8632 93.2192) (width 0.2) (layer "B.Cu") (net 14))
 (segment (start 141.4852 95.6816) (end 143.2763 95.6816) (width 0.2) (layer "F.Cu") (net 22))
 (segment (start 140.1319 96.8052) (end 140.3616 96.8052) (width 0.2) (layer "F.Cu") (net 22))
 (segment (start 150.9325 103.3378) (end 150.9325 103.774) (width 0.2) (layer "F.Cu") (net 22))
 (segment (start 143.2763 95.6816) (end 150.9325 103.3378) (width 0.2) (layer "F.Cu") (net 22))
 (segment (start 140.3616 96.8052) (end 141.4852 95.6816) (width 0.2) (layer "F.Cu") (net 22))
 (segment (start 152.385 103.774) (end 150.9325 103.774) (width 0.2) (layer "F.Cu") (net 22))
 (via (at 140.1319 96.8052) (size 0.6) (drill 0.3) (layers "F.Cu" "B.Cu") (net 22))
 (segment (start 149.352 102.1935) (end 149.352 98.627) (width 0.2) (layer "B.Cu") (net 22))
 (segment (start 138.115 100.838) (end 138.176 100.777) (width 0.2) (layer "B.Cu") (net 22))
 (segment (start 152.385 103.774) (end 150.9325 103.774) (width 0.2) (layer "B.Cu") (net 22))
 (segment (start 138.176 98.5026) (end 139.8734 96.8052) (width 0.2) (layer "B.Cu") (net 22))
 (segment (start 138.176 100.777) (end 138.176 98.627) (width 0.2) (layer "B.Cu") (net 22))
 (segment (start 138.176 98.627) (end 138.176 98.5026) (width 0.2) (layer "B.Cu") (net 22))
 (segment (start 139.8734 96.8052) (end 140.1319 96.8052) (width 0.2) (layer "B.Cu") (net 22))
 (segment (start 150.9325 103.774) (end 149.352 102.1935) (width 0.2) (layer "B.Cu") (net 22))
 (segment (start 154.5126 94.6351) (end 154.5896 94.6351) (width 0.2) (layer "B.Cu") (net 25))
 (segment (start 154.5896 94.6351) (end 156.972 92.2527) (width 0.2) (layer "B.Cu") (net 25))
 (segment (start 156.972 92.2527) (end 156.972 92.127) (width 0.2) (layer "B.Cu") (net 25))
 (segment (start 150.622 98.5257) (end 154.5126 94.6351) (width 0.2) (layer "B.Cu") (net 25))
 (segment (start 150.622 98.627) (end 150.622 98.5257) (width 0.2) (layer "B.Cu") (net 25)))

